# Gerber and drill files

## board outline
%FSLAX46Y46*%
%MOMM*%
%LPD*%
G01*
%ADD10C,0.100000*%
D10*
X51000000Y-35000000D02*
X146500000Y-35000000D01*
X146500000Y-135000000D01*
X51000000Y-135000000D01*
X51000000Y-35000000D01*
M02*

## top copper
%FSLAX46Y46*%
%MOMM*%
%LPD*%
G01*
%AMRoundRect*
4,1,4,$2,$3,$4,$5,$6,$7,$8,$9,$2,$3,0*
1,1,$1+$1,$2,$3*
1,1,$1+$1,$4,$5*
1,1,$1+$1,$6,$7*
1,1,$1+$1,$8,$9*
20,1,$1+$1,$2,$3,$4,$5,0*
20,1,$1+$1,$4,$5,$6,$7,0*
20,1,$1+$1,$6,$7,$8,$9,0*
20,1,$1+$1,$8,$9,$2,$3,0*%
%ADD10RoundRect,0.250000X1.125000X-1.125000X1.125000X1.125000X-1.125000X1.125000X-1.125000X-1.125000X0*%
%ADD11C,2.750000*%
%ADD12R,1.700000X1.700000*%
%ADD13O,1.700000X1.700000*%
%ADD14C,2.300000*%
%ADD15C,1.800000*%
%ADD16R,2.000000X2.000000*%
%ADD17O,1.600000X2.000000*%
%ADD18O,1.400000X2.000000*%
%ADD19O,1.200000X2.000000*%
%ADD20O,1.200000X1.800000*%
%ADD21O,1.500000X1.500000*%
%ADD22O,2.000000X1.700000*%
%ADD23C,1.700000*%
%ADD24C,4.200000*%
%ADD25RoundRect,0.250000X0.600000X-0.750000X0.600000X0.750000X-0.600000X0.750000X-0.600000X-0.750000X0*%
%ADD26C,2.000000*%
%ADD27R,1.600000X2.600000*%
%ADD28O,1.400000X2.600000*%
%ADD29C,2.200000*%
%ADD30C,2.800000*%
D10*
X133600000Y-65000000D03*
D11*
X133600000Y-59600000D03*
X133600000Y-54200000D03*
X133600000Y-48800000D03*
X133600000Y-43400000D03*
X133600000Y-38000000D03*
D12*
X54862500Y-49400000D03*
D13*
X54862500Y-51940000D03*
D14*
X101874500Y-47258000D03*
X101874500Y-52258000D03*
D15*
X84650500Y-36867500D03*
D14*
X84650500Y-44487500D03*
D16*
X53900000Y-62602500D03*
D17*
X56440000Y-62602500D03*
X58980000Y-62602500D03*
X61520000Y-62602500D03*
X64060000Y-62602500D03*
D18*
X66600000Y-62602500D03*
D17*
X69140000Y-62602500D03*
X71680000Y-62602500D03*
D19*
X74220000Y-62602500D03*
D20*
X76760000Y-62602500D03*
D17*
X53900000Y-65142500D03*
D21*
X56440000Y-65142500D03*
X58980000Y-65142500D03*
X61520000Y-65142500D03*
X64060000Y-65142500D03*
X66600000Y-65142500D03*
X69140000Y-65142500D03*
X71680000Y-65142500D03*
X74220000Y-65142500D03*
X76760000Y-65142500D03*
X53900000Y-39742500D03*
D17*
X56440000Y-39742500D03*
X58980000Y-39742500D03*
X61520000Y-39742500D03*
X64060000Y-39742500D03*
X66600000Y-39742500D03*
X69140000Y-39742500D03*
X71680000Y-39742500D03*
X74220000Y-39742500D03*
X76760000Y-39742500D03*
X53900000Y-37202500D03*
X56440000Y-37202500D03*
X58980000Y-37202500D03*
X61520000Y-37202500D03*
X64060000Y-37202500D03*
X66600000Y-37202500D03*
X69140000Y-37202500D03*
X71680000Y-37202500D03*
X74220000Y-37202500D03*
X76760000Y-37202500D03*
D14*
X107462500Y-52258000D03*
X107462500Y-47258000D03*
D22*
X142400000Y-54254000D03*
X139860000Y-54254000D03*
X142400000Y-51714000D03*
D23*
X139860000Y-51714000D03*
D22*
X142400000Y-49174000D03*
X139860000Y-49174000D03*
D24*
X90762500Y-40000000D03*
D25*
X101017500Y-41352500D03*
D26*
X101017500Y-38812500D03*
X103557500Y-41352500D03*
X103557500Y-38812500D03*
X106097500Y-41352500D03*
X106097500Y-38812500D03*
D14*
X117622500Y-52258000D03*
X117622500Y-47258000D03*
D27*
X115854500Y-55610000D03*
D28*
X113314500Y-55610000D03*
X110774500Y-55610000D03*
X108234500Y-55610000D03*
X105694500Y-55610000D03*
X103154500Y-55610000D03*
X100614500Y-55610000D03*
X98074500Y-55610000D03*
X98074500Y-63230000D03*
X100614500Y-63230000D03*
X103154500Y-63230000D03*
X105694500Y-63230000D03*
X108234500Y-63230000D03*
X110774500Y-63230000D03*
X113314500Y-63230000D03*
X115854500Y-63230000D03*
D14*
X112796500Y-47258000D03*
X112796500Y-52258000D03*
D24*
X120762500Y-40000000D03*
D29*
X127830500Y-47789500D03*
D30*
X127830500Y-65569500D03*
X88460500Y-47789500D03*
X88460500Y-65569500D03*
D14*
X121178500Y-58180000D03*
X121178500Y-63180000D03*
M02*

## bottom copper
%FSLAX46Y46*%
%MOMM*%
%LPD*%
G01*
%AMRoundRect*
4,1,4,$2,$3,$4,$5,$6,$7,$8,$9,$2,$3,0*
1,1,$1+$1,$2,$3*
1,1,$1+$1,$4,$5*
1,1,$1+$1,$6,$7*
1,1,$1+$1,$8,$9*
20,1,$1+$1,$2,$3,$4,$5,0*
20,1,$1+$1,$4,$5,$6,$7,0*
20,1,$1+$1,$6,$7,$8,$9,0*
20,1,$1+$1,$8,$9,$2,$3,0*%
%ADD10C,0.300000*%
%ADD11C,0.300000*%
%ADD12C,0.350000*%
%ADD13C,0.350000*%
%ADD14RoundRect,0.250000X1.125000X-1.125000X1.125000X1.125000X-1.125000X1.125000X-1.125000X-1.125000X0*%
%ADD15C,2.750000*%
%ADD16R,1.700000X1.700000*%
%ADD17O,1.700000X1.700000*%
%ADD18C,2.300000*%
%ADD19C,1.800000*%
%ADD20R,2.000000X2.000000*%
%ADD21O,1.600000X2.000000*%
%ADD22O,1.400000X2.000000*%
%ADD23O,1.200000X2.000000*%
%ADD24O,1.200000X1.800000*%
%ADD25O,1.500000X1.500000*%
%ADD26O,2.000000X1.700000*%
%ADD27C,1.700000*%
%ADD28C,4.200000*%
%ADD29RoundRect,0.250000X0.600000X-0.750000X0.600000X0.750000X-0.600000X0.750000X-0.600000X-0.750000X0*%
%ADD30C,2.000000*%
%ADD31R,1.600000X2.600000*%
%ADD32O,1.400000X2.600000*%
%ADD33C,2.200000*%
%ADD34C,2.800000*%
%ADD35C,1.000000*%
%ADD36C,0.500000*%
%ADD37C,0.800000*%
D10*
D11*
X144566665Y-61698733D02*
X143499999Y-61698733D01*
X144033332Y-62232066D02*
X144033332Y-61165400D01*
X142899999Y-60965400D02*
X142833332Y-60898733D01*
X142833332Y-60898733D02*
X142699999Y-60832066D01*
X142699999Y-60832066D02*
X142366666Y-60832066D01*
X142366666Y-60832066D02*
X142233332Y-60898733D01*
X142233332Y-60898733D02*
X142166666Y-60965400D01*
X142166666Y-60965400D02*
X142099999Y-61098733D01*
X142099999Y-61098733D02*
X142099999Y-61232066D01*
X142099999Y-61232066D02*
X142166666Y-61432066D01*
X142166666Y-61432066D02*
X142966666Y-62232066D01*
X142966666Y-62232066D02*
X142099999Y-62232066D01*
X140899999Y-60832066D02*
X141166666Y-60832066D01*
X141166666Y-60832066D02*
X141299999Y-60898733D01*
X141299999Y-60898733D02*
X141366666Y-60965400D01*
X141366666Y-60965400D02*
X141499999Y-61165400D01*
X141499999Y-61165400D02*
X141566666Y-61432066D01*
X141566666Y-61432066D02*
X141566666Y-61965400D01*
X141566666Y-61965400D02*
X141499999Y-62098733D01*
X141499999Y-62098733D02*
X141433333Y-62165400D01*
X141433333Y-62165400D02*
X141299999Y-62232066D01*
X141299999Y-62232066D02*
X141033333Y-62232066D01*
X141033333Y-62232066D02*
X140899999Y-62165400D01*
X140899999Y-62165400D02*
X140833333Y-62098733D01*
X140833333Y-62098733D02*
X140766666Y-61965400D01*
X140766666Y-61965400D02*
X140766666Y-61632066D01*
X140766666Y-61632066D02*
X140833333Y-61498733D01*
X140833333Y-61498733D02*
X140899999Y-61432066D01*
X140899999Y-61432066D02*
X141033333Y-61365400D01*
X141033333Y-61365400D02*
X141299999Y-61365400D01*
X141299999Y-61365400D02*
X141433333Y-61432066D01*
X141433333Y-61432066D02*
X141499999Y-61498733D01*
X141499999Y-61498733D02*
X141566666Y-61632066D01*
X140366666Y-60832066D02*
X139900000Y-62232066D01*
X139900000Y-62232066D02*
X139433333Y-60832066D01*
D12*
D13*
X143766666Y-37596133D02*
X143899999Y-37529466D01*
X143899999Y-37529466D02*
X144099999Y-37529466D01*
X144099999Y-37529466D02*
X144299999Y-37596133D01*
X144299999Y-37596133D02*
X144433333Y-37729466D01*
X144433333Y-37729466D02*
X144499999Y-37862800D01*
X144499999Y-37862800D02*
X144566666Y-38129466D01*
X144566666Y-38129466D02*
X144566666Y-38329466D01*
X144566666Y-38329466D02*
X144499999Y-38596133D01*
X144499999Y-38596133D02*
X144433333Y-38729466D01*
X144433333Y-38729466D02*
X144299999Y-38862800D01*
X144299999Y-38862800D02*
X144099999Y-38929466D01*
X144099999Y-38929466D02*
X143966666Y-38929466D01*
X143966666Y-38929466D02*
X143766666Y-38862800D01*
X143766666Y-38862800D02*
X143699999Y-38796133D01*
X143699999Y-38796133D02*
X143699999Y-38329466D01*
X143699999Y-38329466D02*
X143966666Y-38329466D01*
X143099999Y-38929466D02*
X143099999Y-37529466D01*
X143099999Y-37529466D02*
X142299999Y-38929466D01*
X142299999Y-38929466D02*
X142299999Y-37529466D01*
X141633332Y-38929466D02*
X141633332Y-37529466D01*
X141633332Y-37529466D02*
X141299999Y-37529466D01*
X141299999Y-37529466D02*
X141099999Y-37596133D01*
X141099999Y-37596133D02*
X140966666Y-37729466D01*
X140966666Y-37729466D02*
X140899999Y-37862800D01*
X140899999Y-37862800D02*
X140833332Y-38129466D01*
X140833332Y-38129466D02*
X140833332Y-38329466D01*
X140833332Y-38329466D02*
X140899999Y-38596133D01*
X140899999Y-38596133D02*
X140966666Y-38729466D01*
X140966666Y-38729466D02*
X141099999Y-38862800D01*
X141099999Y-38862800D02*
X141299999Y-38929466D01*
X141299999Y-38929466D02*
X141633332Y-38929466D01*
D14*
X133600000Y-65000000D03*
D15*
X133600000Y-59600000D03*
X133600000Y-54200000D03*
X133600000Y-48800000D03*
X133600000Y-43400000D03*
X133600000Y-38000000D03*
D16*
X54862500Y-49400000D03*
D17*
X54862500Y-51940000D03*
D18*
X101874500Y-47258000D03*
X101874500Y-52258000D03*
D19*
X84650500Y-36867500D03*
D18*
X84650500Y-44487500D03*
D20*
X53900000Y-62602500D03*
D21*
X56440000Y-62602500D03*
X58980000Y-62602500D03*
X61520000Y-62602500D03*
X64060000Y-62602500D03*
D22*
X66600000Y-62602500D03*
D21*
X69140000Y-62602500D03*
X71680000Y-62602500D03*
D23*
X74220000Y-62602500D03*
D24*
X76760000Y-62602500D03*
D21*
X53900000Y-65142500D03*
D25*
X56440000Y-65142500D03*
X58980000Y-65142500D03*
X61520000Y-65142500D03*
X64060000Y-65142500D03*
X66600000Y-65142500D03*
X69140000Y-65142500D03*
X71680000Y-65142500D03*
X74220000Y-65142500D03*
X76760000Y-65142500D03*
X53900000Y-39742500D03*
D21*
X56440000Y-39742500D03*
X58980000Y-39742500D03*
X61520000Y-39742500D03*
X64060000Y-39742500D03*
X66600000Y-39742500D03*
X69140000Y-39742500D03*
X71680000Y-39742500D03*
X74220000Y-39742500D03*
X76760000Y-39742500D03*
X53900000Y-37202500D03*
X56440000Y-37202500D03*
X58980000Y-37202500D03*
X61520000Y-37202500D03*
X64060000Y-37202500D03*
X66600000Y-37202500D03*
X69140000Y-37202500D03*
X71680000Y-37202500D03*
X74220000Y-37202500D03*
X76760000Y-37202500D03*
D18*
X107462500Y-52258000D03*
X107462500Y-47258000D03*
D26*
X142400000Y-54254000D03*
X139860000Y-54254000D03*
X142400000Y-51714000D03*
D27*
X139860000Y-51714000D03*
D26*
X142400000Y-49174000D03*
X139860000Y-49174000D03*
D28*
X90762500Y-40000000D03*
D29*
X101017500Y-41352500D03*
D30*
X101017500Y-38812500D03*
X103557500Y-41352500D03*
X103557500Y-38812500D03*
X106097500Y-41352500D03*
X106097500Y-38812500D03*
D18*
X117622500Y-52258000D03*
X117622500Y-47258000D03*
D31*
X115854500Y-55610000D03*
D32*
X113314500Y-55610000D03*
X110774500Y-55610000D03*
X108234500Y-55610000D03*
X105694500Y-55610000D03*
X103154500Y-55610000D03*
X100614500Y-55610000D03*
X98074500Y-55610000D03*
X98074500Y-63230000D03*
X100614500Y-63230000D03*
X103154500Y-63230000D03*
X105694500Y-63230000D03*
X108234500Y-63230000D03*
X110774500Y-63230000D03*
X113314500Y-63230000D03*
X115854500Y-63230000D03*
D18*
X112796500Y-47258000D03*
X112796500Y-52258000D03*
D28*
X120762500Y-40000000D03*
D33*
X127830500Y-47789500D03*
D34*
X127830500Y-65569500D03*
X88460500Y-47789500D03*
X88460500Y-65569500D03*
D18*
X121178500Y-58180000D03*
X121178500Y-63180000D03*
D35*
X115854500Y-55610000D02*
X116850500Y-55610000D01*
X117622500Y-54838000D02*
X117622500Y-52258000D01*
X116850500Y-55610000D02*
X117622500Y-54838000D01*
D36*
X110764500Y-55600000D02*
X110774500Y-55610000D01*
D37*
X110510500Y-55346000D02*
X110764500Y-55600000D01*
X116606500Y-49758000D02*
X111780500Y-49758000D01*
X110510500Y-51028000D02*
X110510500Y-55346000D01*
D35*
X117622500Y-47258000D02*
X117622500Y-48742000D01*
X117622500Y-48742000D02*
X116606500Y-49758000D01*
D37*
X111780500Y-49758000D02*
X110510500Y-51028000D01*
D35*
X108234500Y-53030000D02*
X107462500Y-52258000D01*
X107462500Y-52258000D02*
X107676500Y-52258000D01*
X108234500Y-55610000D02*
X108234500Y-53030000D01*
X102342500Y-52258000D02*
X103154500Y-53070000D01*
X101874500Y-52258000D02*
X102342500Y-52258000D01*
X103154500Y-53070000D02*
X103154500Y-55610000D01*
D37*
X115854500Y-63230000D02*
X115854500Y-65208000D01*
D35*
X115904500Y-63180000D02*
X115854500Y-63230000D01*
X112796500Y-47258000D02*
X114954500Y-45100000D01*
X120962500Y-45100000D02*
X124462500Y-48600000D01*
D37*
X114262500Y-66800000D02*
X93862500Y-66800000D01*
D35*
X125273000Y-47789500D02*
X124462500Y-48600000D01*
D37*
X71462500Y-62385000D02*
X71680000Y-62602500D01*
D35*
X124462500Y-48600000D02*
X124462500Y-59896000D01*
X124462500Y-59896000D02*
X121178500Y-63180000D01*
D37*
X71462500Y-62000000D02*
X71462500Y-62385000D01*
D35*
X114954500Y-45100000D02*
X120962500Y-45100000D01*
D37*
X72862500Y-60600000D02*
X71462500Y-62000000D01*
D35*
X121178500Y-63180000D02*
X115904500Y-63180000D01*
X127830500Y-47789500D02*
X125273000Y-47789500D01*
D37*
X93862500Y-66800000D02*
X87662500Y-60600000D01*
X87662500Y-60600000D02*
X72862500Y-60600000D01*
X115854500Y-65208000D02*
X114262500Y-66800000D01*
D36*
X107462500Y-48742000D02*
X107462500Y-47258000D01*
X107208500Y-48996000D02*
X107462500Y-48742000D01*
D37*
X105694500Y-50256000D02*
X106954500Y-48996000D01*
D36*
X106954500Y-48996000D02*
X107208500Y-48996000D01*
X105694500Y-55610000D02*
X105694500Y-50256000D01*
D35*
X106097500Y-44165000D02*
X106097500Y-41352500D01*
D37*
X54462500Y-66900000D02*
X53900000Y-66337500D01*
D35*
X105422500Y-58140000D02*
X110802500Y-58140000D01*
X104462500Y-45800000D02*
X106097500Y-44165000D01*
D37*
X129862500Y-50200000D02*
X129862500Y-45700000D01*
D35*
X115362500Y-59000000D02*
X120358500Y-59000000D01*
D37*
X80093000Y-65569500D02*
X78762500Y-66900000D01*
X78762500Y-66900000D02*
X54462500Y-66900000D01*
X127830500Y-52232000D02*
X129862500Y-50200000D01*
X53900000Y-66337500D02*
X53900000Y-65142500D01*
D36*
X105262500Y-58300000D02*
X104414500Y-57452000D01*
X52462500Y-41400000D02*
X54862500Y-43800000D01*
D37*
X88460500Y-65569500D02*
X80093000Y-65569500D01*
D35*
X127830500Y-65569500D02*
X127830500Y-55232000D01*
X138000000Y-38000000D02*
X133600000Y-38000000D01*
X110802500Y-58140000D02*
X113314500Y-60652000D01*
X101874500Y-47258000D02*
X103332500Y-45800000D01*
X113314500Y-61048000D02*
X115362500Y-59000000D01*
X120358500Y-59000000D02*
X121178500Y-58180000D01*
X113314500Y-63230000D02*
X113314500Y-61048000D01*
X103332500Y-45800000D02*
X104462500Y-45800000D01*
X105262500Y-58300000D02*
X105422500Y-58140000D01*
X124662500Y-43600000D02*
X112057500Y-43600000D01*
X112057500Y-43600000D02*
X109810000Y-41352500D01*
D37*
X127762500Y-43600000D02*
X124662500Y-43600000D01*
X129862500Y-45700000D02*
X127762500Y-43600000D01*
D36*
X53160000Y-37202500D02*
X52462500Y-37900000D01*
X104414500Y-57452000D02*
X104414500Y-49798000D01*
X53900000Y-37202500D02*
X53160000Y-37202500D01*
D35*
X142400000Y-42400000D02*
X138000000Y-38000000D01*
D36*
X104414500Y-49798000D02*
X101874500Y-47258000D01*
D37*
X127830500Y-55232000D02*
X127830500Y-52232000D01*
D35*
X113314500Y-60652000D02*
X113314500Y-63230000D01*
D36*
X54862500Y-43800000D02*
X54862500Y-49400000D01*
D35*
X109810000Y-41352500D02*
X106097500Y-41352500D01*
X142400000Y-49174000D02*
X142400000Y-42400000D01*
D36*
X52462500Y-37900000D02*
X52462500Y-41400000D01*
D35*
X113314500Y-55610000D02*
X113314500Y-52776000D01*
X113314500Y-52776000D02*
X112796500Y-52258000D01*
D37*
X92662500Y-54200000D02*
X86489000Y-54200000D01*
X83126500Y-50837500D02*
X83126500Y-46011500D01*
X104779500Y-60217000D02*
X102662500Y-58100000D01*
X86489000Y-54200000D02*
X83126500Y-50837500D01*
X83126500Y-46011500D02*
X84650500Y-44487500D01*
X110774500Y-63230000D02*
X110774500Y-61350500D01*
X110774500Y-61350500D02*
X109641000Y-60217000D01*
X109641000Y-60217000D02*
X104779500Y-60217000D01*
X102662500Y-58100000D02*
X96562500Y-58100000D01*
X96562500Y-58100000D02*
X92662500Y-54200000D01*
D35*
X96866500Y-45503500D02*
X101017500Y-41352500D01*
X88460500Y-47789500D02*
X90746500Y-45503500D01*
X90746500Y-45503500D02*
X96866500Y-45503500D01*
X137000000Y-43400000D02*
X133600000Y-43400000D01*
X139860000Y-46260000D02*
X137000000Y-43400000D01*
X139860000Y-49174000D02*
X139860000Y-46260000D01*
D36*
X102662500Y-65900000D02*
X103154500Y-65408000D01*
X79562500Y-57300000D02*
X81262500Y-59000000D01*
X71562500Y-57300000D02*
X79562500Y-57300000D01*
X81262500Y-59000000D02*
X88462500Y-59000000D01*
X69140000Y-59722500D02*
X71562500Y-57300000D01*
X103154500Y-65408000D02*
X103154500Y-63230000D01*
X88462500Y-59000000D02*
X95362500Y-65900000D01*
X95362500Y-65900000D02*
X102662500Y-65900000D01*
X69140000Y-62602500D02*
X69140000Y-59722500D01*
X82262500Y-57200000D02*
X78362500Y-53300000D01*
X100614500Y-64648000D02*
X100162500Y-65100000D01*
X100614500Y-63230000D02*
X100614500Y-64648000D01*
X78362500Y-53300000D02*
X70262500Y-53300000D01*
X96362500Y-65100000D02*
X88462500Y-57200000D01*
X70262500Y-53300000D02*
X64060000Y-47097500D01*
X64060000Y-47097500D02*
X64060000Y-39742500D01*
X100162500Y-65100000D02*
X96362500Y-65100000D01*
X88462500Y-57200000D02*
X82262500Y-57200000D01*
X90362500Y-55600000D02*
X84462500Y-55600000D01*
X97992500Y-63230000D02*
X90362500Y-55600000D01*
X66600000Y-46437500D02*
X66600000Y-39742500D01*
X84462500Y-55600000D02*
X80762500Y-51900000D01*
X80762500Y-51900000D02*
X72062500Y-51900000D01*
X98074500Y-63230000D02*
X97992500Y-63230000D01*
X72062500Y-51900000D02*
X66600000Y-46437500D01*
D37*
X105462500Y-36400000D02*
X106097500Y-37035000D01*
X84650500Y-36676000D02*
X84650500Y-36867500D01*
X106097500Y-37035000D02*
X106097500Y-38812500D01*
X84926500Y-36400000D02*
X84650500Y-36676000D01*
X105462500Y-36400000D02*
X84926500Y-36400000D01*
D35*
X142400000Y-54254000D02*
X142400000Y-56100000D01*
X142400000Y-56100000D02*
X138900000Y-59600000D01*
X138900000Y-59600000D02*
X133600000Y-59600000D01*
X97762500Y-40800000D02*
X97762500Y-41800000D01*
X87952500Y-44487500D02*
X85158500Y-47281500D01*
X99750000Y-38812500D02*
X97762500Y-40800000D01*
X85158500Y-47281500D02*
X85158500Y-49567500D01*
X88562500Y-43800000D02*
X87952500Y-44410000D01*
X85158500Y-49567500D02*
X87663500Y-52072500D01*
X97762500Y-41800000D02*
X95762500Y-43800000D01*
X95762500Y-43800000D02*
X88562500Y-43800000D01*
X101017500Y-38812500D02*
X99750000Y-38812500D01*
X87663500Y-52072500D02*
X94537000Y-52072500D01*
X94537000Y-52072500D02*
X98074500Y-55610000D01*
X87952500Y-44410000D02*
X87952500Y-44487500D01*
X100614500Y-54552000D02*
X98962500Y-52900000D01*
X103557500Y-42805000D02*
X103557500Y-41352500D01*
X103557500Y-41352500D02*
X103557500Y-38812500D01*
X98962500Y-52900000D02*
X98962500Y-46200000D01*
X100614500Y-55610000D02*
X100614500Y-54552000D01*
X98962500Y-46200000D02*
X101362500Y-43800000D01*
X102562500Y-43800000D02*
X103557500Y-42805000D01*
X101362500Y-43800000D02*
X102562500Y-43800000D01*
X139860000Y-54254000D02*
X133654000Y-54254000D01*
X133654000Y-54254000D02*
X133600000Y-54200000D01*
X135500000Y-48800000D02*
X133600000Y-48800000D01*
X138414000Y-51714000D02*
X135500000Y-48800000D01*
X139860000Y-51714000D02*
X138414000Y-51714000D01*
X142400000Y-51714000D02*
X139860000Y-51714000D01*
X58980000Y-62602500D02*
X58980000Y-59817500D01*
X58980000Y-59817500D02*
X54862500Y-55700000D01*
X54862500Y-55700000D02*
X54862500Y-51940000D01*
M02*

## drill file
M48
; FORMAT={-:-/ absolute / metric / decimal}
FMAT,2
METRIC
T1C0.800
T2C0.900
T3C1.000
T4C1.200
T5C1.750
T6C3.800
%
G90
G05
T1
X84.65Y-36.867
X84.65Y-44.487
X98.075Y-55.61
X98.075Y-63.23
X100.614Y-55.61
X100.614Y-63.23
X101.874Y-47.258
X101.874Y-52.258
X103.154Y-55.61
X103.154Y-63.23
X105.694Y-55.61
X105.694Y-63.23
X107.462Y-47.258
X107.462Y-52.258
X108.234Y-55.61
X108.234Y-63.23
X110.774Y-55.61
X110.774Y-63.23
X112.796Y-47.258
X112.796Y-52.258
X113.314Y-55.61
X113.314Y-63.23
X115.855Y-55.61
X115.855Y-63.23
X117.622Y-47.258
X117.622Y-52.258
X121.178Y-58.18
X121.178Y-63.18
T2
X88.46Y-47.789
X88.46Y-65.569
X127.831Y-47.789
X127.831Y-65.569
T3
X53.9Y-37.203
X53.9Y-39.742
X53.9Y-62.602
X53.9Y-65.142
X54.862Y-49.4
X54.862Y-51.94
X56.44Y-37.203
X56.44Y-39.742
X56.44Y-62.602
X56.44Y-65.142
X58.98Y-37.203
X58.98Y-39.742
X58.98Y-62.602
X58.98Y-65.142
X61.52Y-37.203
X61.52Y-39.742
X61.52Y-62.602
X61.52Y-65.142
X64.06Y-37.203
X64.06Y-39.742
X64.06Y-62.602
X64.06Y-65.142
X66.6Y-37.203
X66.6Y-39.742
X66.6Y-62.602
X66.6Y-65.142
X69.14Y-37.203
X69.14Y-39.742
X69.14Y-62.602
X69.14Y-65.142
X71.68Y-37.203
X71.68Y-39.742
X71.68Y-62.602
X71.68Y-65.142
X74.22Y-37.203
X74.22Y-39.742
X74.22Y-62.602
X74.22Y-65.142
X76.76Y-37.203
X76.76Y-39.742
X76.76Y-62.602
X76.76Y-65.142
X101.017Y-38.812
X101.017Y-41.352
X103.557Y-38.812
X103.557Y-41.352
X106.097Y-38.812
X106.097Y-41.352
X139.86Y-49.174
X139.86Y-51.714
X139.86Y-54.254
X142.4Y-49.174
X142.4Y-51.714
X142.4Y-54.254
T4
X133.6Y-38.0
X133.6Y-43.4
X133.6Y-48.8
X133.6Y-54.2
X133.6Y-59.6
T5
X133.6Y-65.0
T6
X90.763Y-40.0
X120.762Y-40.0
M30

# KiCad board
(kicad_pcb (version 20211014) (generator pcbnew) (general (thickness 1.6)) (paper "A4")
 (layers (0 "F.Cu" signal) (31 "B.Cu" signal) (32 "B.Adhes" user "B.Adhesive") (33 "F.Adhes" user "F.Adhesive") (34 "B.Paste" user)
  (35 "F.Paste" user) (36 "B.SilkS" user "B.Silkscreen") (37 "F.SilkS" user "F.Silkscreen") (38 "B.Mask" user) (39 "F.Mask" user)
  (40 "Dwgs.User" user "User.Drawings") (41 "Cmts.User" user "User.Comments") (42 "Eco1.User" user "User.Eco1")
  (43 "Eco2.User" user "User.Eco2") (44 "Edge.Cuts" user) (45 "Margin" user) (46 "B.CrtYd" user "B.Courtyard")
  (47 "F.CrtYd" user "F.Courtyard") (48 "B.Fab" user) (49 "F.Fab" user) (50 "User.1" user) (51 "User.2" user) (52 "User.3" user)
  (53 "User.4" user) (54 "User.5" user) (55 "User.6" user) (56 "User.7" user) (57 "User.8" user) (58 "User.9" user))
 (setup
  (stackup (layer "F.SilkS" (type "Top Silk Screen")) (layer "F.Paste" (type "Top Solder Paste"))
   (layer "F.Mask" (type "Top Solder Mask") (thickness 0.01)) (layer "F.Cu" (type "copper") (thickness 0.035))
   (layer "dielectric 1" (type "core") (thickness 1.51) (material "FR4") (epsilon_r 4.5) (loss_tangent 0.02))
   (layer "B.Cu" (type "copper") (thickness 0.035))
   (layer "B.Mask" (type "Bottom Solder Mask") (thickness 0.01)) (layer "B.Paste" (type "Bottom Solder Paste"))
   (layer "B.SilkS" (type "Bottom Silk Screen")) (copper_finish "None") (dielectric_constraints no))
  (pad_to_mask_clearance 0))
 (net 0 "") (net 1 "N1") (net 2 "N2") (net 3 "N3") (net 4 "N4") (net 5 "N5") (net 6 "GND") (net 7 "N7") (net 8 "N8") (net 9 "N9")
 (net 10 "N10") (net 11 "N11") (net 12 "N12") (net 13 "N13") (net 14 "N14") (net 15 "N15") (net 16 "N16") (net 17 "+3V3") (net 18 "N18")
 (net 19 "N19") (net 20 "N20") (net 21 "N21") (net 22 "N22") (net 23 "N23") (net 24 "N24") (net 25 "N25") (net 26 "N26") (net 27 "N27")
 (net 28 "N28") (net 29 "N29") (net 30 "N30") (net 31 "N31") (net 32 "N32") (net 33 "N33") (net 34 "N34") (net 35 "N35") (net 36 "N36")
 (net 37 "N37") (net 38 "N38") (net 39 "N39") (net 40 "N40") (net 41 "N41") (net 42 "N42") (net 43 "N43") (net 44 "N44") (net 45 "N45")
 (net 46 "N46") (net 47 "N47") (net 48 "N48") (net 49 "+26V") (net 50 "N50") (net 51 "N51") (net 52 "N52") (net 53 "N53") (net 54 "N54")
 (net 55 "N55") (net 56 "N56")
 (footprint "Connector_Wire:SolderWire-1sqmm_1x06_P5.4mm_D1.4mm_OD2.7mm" (layer "F.Cu") (at 133.6 65 90)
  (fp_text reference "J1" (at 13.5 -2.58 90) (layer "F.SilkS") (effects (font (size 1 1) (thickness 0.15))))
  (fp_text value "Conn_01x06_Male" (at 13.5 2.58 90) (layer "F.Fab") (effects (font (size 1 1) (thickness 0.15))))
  (pad "1" thru_hole roundrect (at 0 0 90) (size 2.75 2.75) (drill 1.75) (layers *.Cu *.Mask) (roundrect_rratio 0.090909) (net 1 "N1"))
  (pad "2" thru_hole circle (at 5.4 0 90) (size 2.75 2.75) (drill 1.2) (layers *.Cu *.Mask) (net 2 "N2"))
  (pad "3" thru_hole circle (at 10.8 0 90) (size 2.75 2.75) (drill 1.2) (layers *.Cu *.Mask) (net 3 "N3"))
  (pad "4" thru_hole circle (at 16.2 0 90) (size 2.75 2.75) (drill 1.2) (layers *.Cu *.Mask) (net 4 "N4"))
  (pad "5" thru_hole circle (at 21.6 0 90) (size 2.75 2.75) (drill 1.2) (layers *.Cu *.Mask) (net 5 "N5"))
  (pad "6" thru_hole circle (at 27 0 90) (size 2.75 2.75) (drill 1.2) (layers *.Cu *.Mask) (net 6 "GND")))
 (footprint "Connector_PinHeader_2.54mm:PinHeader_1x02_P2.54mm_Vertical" (layer "F.Cu") (at 54.8625 49.4)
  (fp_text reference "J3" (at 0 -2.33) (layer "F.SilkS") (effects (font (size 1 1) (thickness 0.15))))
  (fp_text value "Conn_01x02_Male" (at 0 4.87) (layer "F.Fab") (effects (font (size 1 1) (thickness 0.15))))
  (pad "1" thru_hole rect (at 0 0) (size 1.7 1.7) (drill 1) (layers *.Cu *.Mask) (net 6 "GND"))
  (pad "2" thru_hole oval (at 0 2.54) (size 1.7 1.7) (drill 1) (layers *.Cu *.Mask) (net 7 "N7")))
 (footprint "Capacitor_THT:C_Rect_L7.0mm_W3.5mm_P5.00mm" (layer "F.Cu") (at 101.8745 47.258 -90)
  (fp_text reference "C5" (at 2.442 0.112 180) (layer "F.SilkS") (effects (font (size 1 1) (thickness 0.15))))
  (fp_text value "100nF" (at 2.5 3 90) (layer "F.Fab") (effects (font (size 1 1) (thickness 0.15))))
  (pad "1" thru_hole circle (at 0 0 270) (size 2.3 2.3) (drill 0.8) (layers *.Cu *.Mask) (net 6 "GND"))
  (pad "2" thru_hole circle (at 5 0 270) (size 2.3 2.3) (drill 0.8) (layers *.Cu *.Mask) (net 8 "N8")))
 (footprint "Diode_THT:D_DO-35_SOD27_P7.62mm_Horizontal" (layer "F.Cu") (at 84.6505 36.8675 -90)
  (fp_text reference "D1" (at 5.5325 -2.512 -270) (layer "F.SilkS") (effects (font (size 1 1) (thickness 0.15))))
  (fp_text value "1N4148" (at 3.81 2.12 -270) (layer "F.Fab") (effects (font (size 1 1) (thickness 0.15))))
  (pad "1" thru_hole circle (at 0 0 270) (size 1.8 1.8) (drill 0.8) (layers *.Cu *.Mask) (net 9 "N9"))
  (pad "2" thru_hole circle (at 7.62 0 270) (size 2.3 2.3) (drill 0.8) (layers *.Cu *.Mask) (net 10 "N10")))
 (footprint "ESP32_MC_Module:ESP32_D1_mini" (layer "F.Cu") (at 53.9 65.1425 90)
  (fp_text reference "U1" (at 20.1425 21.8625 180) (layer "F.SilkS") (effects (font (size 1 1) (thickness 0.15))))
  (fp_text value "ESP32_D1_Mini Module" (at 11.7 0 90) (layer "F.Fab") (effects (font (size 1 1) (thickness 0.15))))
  (pad "1" thru_hole rect (at 2.54 0 90) (size 2 2) (drill 1) (layers *.Cu *.Mask) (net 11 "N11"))
  (pad "2" thru_hole oval (at 2.54 2.54 90) (size 2 1.6) (drill 1) (layers *.Cu *.Mask) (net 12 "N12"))
  (pad "3" thru_hole oval (at 2.54 5.08 90) (size 2 1.6) (drill 1) (layers *.Cu *.Mask) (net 7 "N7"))
  (pad "4" thru_hole oval (at 2.54 7.62 90) (size 2 1.6) (drill 1) (layers *.Cu *.Mask) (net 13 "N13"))
  (pad "5" thru_hole oval (at 2.54 10.16 90) (size 2 1.6) (drill 1) (layers *.Cu *.Mask) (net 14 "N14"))
  (pad "6" thru_hole oval (at 2.54 12.7 90) (size 2 1.4) (drill 1) (layers *.Cu *.Mask) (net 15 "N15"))
  (pad "7" thru_hole oval (at 2.54 15.24 90) (size 2 1.6) (drill 1) (layers *.Cu *.Mask) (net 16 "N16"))
  (pad "8" thru_hole oval (at 2.54 17.78 90) (size 2 1.6) (drill 1) (layers *.Cu *.Mask) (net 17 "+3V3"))
  (pad "9" thru_hole oval (at 2.54 20.32 90) (size 2 1.2) (drill 1) (layers *.Cu *.Mask) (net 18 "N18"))
  (pad "10" thru_hole oval (at 2.54 22.86 90) (size 1.8 1.2) (drill 1) (layers *.Cu *.Mask) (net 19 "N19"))
  (pad "11" thru_hole oval (at 0 0 90) (size 2 1.6) (drill 1) (layers *.Cu *.Mask) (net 6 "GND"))
  (pad "12" thru_hole oval (at 0 2.54 90) (size 1.5 1.5) (drill 1) (layers *.Cu *.Mask) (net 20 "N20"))
  (pad "13" thru_hole oval (at 0 5.08 90) (size 1.5 1.5) (drill 1) (layers *.Cu *.Mask) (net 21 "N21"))
  (pad "14" thru_hole oval (at 0 7.62 90) (size 1.5 1.5) (drill 1) (layers *.Cu *.Mask) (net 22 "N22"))
  (pad "15" thru_hole oval (at 0 10.16 90) (size 1.5 1.5) (drill 1) (layers *.Cu *.Mask) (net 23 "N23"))
  (pad "16" thru_hole oval (at 0 12.7 90) (size 1.5 1.5) (drill 1) (layers *.Cu *.Mask) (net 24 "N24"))
  (pad "17" thru_hole oval (at 0 15.24 90) (size 1.5 1.5) (drill 1) (layers *.Cu *.Mask) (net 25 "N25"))
  (pad "18" thru_hole oval (at 0 17.78 90) (size 1.5 1.5) (drill 1) (layers *.Cu *.Mask) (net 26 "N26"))
  (pad "19" thru_hole oval (at 0 20.32 90) (size 1.5 1.5) (drill 1) (layers *.Cu *.Mask) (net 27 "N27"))
  (pad "20" thru_hole oval (at 0 22.86 90) (size 1.5 1.5) (drill 1) (layers *.Cu *.Mask) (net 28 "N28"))
  (pad "21" thru_hole oval (at 25.4 0 90) (size 1.5 1.5) (drill 1) (layers *.Cu *.Mask) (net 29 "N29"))
  (pad "22" thru_hole oval (at 25.4 2.54 90) (size 2 1.6) (drill 1) (layers *.Cu *.Mask) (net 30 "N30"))
  (pad "23" thru_hole oval (at 25.4 5.08 90) (size 2 1.6) (drill 1) (layers *.Cu *.Mask) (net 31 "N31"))
  (pad "24" thru_hole oval (at 25.4 7.62 90) (size 2 1.6) (drill 1) (layers *.Cu *.Mask) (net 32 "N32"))
  (pad "25" thru_hole oval (at 25.4 10.16 90) (size 2 1.6) (drill 1) (layers *.Cu *.Mask) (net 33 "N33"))
  (pad "26" thru_hole oval (at 25.4 12.7 90) (size 2 1.6) (drill 1) (layers *.Cu *.Mask) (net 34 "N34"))
  (pad "27" thru_hole oval (at 25.4 15.24 90) (size 2 1.6) (drill 1) (layers *.Cu *.Mask) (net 6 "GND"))
  (pad "28" thru_hole oval (at 25.4 17.78 90) (size 2 1.6) (drill 1) (layers *.Cu *.Mask) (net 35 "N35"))
  (pad "29" thru_hole oval (at 25.4 20.32 90) (size 2 1.6) (drill 1) (layers *.Cu *.Mask) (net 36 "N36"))
  (pad "30" thru_hole oval (at 25.4 22.86 90) (size 2 1.6) (drill 1) (layers *.Cu *.Mask) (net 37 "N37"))
  (pad "31" thru_hole oval (at 27.94 0 90) (size 2 1.6) (drill 1) (layers *.Cu *.Mask) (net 6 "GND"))
  (pad "32" thru_hole oval (at 27.94 2.54 90) (size 2 1.6) (drill 1) (layers *.Cu *.Mask) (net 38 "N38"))
  (pad "33" thru_hole oval (at 27.94 5.08 90) (size 2 1.6) (drill 1) (layers *.Cu *.Mask) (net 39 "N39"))
  (pad "34" thru_hole oval (at 27.94 7.62 90) (size 2 1.6) (drill 1) (layers *.Cu *.Mask) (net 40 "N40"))
  (pad "35" thru_hole oval (at 27.94 10.16 90) (size 2 1.6) (drill 1) (layers *.Cu *.Mask) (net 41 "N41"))
  (pad "36" thru_hole oval (at 27.94 12.7 90) (size 2 1.6) (drill 1) (layers *.Cu *.Mask) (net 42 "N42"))
  (pad "37" thru_hole oval (at 27.94 15.24 90) (size 2 1.6) (drill 1) (layers *.Cu *.Mask) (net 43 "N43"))
  (pad "38" thru_hole oval (at 27.94 17.78 90) (size 2 1.6) (drill 1) (layers *.Cu *.Mask) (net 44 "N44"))
  (pad "39" thru_hole oval (at 27.94 20.32 90) (size 2 1.6) (drill 1) (layers *.Cu *.Mask) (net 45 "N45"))
  (pad "40" thru_hole oval (at 27.94 22.86 90) (size 2 1.6) (drill 1) (layers *.Cu *.Mask) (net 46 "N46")))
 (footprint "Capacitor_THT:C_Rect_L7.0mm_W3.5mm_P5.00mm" (layer "F.Cu") (at 107.4625 52.258 90)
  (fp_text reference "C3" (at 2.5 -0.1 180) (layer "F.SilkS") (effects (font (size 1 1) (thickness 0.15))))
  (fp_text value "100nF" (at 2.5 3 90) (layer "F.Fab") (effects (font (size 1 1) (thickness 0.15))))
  (pad "1" thru_hole circle (at 0 0 90) (size 2.3 2.3) (drill 0.8) (layers *.Cu *.Mask) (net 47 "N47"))
  (pad "2" thru_hole circle (at 5 0 90) (size 2.3 2.3) (drill 0.8) (layers *.Cu *.Mask) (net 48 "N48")))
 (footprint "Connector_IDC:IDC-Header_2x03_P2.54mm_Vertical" (layer "F.Cu") (at 142.4 54.254 180)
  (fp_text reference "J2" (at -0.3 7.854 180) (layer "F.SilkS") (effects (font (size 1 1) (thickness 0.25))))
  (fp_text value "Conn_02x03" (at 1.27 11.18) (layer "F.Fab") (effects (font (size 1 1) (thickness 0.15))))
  (pad "1" thru_hole oval (at 0 0 180) (size 2 1.7) (drill 1) (layers *.Cu *.Mask) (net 2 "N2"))
  (pad "2" thru_hole oval (at 2.54 0 180) (size 2 1.7) (drill 1) (layers *.Cu *.Mask) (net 3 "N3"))
  (pad "3" thru_hole oval (at 0 2.54 180) (size 2 1.7) (drill 1) (layers *.Cu *.Mask) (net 4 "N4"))
  (pad "4" thru_hole circle (at 2.54 2.54 180) (size 1.7 1.7) (drill 1) (layers *.Cu *.Mask) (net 4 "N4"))
  (pad "5" thru_hole oval (at 0 5.08 180) (size 2 1.7) (drill 1) (layers *.Cu *.Mask) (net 6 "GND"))
  (pad "6" thru_hole oval (at 2.54 5.08 180) (size 2 1.7) (drill 1) (layers *.Cu *.Mask) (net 5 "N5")))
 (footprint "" (layer "F.Cu") (at 90.7625 40)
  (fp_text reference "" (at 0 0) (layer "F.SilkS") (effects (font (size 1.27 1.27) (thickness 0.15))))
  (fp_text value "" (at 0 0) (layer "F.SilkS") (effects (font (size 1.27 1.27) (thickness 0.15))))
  (pad "1" thru_hole circle (at 0 0 270) (size 4.2 4.2) (drill 3.8) (layers *.Cu *.Mask) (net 17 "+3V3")))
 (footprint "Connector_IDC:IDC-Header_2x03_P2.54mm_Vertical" (layer "F.Cu") (at 101.0175 41.3525 90)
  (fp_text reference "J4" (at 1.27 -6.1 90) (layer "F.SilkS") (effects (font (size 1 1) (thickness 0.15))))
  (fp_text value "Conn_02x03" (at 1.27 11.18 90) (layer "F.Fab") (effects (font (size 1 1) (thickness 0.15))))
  (pad "1" thru_hole roundrect (at 0 0 90) (size 2 1.7) (drill 1) (layers *.Cu *.Mask) (roundrect_rratio 0.147059) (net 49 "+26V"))
  (pad "2" thru_hole circle (at 2.54 0 90) (size 2 2) (drill 1) (layers *.Cu *.Mask) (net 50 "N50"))
  (pad "3" thru_hole circle (at 0 2.54 90) (size 2 2) (drill 1) (layers *.Cu *.Mask) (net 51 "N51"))
  (pad "4" thru_hole circle (at 2.54 2.54 90) (size 2 2) (drill 1) (layers *.Cu *.Mask) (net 51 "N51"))
  (pad "5" thru_hole circle (at 0 5.08 90) (size 2 2) (drill 1) (layers *.Cu *.Mask) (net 6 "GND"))
  (pad "6" thru_hole circle (at 2.54 5.08 90) (size 2 2) (drill 1) (layers *.Cu *.Mask) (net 9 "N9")))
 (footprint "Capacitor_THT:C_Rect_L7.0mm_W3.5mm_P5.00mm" (layer "F.Cu") (at 117.6225 52.258 90)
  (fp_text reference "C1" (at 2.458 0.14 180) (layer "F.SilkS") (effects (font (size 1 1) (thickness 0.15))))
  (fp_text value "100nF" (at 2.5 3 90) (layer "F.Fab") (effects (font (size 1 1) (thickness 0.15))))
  (pad "1" thru_hole circle (at 0 0 90) (size 2.3 2.3) (drill 0.8) (layers *.Cu *.Mask) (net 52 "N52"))
  (pad "2" thru_hole circle (at 5 0 90) (size 2.3 2.3) (drill 0.8) (layers *.Cu *.Mask) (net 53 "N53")))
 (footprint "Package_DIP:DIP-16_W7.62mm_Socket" (layer "F.Cu") (at 115.8545 55.61 -90)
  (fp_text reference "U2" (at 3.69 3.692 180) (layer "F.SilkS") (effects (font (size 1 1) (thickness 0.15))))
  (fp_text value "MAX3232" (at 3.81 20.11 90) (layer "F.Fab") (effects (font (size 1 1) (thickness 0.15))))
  (pad "1" thru_hole rect (at 0 0 270) (size 2.6 1.6) (drill 0.8) (layers *.Cu *.Mask) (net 52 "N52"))
  (pad "2" thru_hole oval (at 0 2.54 270) (size 2.6 1.4) (drill 0.8) (layers *.Cu *.Mask) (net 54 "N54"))
  (pad "3" thru_hole oval (at 0 5.08 270) (size 2.6 1.4) (drill 0.8) (layers *.Cu *.Mask) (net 53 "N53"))
  (pad "4" thru_hole oval (at 0 7.62 270) (size 2.6 1.4) (drill 0.8) (layers *.Cu *.Mask) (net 47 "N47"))
  (pad "5" thru_hole oval (at 0 10.16 270) (size 2.6 1.4) (drill 0.8) (layers *.Cu *.Mask) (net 48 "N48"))
  (pad "6" thru_hole oval (at 0 12.7 270) (size 2.6 1.4) (drill 0.8) (layers *.Cu *.Mask) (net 8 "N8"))
  (pad "7" thru_hole oval (at 0 15.24 270) (size 2.6 1.4) (drill 0.8) (layers *.Cu *.Mask) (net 51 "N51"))
  (pad "8" thru_hole oval (at 0 17.78 270) (size 2.6 1.4) (drill 0.8) (layers *.Cu *.Mask) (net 50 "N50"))
  (pad "9" thru_hole oval (at 7.62 17.78 270) (size 2.6 1.4) (drill 0.8) (layers *.Cu *.Mask) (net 34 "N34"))
  (pad "10" thru_hole oval (at 7.62 15.24 270) (size 2.6 1.4) (drill 0.8) (layers *.Cu *.Mask) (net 33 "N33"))
  (pad "11" thru_hole oval (at 7.62 12.7 270) (size 2.6 1.4) (drill 0.8) (layers *.Cu *.Mask) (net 16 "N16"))
  (pad "12" thru_hole oval (at 7.62 10.16 270) (size 2.6 1.4) (drill 0.8) (layers *.Cu *.Mask) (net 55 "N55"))
  (pad "13" thru_hole oval (at 7.62 7.62 270) (size 2.6 1.4) (drill 0.8) (layers *.Cu *.Mask) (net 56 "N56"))
  (pad "14" thru_hole oval (at 7.62 5.08 270) (size 2.6 1.4) (drill 0.8) (layers *.Cu *.Mask) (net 10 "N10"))
  (pad "15" thru_hole oval (at 7.62 2.54 270) (size 2.6 1.4) (drill 0.8) (layers *.Cu *.Mask) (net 6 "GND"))
  (pad "16" thru_hole oval (at 7.62 0 270) (size 2.6 1.4) (drill 0.8) (layers *.Cu *.Mask) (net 17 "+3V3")))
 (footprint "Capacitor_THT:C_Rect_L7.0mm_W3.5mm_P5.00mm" (layer "F.Cu") (at 112.7965 47.258 -90)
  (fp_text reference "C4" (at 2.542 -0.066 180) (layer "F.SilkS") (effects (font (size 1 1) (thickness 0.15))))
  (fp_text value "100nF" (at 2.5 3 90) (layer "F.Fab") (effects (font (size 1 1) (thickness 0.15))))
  (pad "1" thru_hole circle (at 0 0 270) (size 2.3 2.3) (drill 0.8) (layers *.Cu *.Mask) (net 17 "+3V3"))
  (pad "2" thru_hole circle (at 5 0 270) (size 2.3 2.3) (drill 0.8) (layers *.Cu *.Mask) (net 54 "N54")))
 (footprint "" (layer "F.Cu") (at 120.7625 40)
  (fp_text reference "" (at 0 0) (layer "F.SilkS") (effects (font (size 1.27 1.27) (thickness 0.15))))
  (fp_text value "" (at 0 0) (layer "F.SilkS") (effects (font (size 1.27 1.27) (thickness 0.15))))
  (pad "1" thru_hole circle (at 0 0 270) (size 4.2 4.2) (drill 3.8) (layers *.Cu *.Mask) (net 17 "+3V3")))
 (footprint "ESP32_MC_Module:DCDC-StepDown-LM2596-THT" (layer "F.Cu") (at 127.8305 47.7895 -90)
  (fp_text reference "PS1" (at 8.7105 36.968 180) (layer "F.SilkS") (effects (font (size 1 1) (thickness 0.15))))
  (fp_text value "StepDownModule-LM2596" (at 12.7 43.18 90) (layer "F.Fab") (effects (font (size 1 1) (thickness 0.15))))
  (pad "1" thru_hole circle (at 0 0 270) (size 2.2 2.2) (drill 0.9) (layers *.Cu *.Mask) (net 17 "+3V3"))
  (pad "2" thru_hole circle (at 17.78 0 270) (size 2.8 2.8) (drill 0.9) (layers *.Cu *.Mask) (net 6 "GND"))
  (pad "3" thru_hole circle (at 0 39.37 270) (size 2.8 2.8) (drill 0.9) (layers *.Cu *.Mask) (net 49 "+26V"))
  (pad "4" thru_hole circle (at 17.78 39.37 270) (size 2.8 2.8) (drill 0.9) (layers *.Cu *.Mask) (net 6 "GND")))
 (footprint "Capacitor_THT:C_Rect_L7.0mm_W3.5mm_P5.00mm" (layer "F.Cu") (at 121.1785 58.18 -90)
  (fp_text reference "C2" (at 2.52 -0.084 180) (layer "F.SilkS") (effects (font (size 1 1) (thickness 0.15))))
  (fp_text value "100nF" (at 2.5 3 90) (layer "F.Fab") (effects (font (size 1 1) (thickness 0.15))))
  (pad "1" thru_hole circle (at 0 0 270) (size 2.3 2.3) (drill 0.8) (layers *.Cu *.Mask) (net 6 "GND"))
  (pad "2" thru_hole circle (at 5 0 270) (size 2.3 2.3) (drill 0.8) (layers *.Cu *.Mask) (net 17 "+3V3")))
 (gr_rect (start 51 35) (end 146.5 135) (layer "Edge.Cuts") (width 0.1) (fill none))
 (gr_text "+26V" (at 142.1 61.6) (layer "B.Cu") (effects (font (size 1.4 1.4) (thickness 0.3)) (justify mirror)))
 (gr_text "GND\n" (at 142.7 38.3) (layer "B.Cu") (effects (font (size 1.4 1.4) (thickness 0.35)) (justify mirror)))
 (segment (start 115.8545 55.61) (end 116.8505 55.61) (width 1) (layer "B.Cu") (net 52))
 (segment (start 117.6225 54.838) (end 117.6225 52.258) (width 1) (layer "B.Cu") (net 52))
 (segment (start 116.8505 55.61) (end 117.6225 54.838) (width 1) (layer "B.Cu") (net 52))
 (segment (start 110.7645 55.6) (end 110.7745 55.61) (width 0.5) (layer "B.Cu") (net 53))
 (segment (start 110.5105 55.346) (end 110.7645 55.6) (width 0.8) (layer "B.Cu") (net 53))
 (segment (start 116.6065 49.758) (end 111.7805 49.758) (width 0.8) (layer "B.Cu") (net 53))
 (segment (start 110.5105 51.028) (end 110.5105 55.346) (width 0.8) (layer "B.Cu") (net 53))
 (segment (start 117.6225 47.258) (end 117.6225 48.742) (width 1) (layer "B.Cu") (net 53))
 (segment (start 117.6225 48.742) (end 116.6065 49.758) (width 1) (layer "B.Cu") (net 53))
 (segment (start 111.7805 49.758) (end 110.5105 51.028) (width 0.8) (layer "B.Cu") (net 53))
 (segment (start 108.2345 53.03) (end 107.4625 52.258) (width 1) (layer "B.Cu") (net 47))
 (segment (start 107.4625 52.258) (end 107.6765 52.258) (width 1) (layer "B.Cu") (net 47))
 (segment (start 108.2345 55.61) (end 108.2345 53.03) (width 1) (layer "B.Cu") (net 47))
 (segment (start 102.3425 52.258) (end 103.1545 53.07) (width 1) (layer "B.Cu") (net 8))
 (segment (start 101.8745 52.258) (end 102.3425 52.258) (width 1) (layer "B.Cu") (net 8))
 (segment (start 103.1545 53.07) (end 103.1545 55.61) (width 1) (layer "B.Cu") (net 8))
 (segment (start 115.8545 63.23) (end 115.8545 65.208) (width 0.8) (layer "B.Cu") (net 17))
 (segment (start 115.9045 63.18) (end 115.8545 63.23) (width 1) (layer "B.Cu") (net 17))
 (segment (start 112.7965 47.258) (end 114.9545 45.1) (width 1) (layer "B.Cu") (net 17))
 (segment (start 120.9625 45.1) (end 124.4625 48.6) (width 1) (layer "B.Cu") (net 17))
 (segment (start 114.2625 66.8) (end 93.8625 66.8) (width 0.8) (layer "B.Cu") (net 17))
 (segment (start 125.273 47.7895) (end 124.4625 48.6) (width 1) (layer "B.Cu") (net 17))
 (segment (start 71.4625 62.385) (end 71.68 62.6025) (width 0.8) (layer "B.Cu") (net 17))
 (segment (start 124.4625 48.6) (end 124.4625 59.896) (width 1) (layer "B.Cu") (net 17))
 (segment (start 124.4625 59.896) (end 121.1785 63.18) (width 1) (layer "B.Cu") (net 17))
 (segment (start 71.4625 62) (end 71.4625 62.385) (width 0.8) (layer "B.Cu") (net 17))
 (segment (start 114.9545 45.1) (end 120.9625 45.1) (width 1) (layer "B.Cu") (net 17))
 (segment (start 72.8625 60.6) (end 71.4625 62) (width 0.8) (layer "B.Cu") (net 17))
 (segment (start 121.1785 63.18) (end 115.9045 63.18) (width 1) (layer "B.Cu") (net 17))
 (segment (start 127.8305 47.7895) (end 125.273 47.7895) (width 1) (layer "B.Cu") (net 17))
 (segment (start 93.8625 66.8) (end 87.6625 60.6) (width 0.8) (layer "B.Cu") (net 17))
 (segment (start 87.6625 60.6) (end 72.8625 60.6) (width 0.8) (layer "B.Cu") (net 17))
 (segment (start 115.8545 65.208) (end 114.2625 66.8) (width 0.8) (layer "B.Cu") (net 17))
 (segment (start 107.4625 48.742) (end 107.4625 47.258) (width 0.5) (layer "B.Cu") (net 48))
 (segment (start 107.2085 48.996) (end 107.4625 48.742) (width 0.5) (layer "B.Cu") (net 48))
 (segment (start 105.6945 50.256) (end 106.9545 48.996) (width 0.8) (layer "B.Cu") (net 48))
 (segment (start 106.9545 48.996) (end 107.2085 48.996) (width 0.5) (layer "B.Cu") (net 48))
 (segment (start 105.6945 55.61) (end 105.6945 50.256) (width 0.5) (layer "B.Cu") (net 48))
 (segment (start 106.0975 44.165) (end 106.0975 41.3525) (width 1) (layer "B.Cu") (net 6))
 (segment (start 54.4625 66.9) (end 53.9 66.3375) (width 0.8) (layer "B.Cu") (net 6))
 (segment (start 105.4225 58.14) (end 110.8025 58.14) (width 1) (layer "B.Cu") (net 6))
 (segment (start 104.4625 45.8) (end 106.0975 44.165) (width 1) (layer "B.Cu") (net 6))
 (segment (start 129.8625 50.2) (end 129.8625 45.7) (width 0.8) (layer "B.Cu") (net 6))
 (segment (start 115.3625 59) (end 120.3585 59) (width 1) (layer "B.Cu") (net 6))
 (segment (start 80.093 65.5695) (end 78.7625 66.9) (width 0.8) (layer "B.Cu") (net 6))
 (segment (start 78.7625 66.9) (end 54.4625 66.9) (width 0.8) (layer "B.Cu") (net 6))
 (segment (start 127.8305 52.232) (end 129.8625 50.2) (width 0.8) (layer "B.Cu") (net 6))
 (segment (start 53.9 66.3375) (end 53.9 65.1425) (width 0.8) (layer "B.Cu") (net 6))
 (segment (start 105.2625 58.3) (end 104.4145 57.452) (width 0.5) (layer "B.Cu") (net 6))
 (segment (start 52.4625 41.4) (end 54.8625 43.8) (width 0.5) (layer "B.Cu") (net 6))
 (segment (start 88.4605 65.5695) (end 80.093 65.5695) (width 0.8) (layer "B.Cu") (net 6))
 (segment (start 127.8305 65.5695) (end 127.8305 55.232) (width 1) (layer "B.Cu") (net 6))
 (segment (start 138 38) (end 133.6 38) (width 1) (layer "B.Cu") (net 6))
 (segment (start 110.8025 58.14) (end 113.3145 60.652) (width 1) (layer "B.Cu") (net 6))
 (segment (start 101.8745 47.258) (end 103.3325 45.8) (width 1) (layer "B.Cu") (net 6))
 (segment (start 113.3145 61.048) (end 115.3625 59) (width 1) (layer "B.Cu") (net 6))
 (segment (start 120.3585 59) (end 121.1785 58.18) (width 1) (layer "B.Cu") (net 6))
 (segment (start 113.3145 63.23) (end 113.3145 61.048) (width 1) (layer "B.Cu") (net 6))
 (segment (start 103.3325 45.8) (end 104.4625 45.8) (width 1) (layer "B.Cu") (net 6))
 (segment (start 105.2625 58.3) (end 105.4225 58.14) (width 1) (layer "B.Cu") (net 6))
 (segment (start 124.6625 43.6) (end 112.0575 43.6) (width 1) (layer "B.Cu") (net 6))
 (segment (start 112.0575 43.6) (end 109.81 41.3525) (width 1) (layer "B.Cu") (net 6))
 (segment (start 127.7625 43.6) (end 124.6625 43.6) (width 0.8) (layer "B.Cu") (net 6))
 (segment (start 129.8625 45.7) (end 127.7625 43.6) (width 0.8) (layer "B.Cu") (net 6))
 (segment (start 53.16 37.2025) (end 52.4625 37.9) (width 0.5) (layer "B.Cu") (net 6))
 (segment (start 104.4145 57.452) (end 104.4145 49.798) (width 0.5) (layer "B.Cu") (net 6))
 (segment (start 53.9 37.2025) (end 53.16 37.2025) (width 0.5) (layer "B.Cu") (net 6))
 (segment (start 142.4 42.4) (end 138 38) (width 1) (layer "B.Cu") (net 6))
 (segment (start 104.4145 49.798) (end 101.8745 47.258) (width 0.5) (layer "B.Cu") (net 6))
 (segment (start 127.8305 55.232) (end 127.8305 52.232) (width 0.8) (layer "B.Cu") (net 6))
 (segment (start 113.3145 60.652) (end 113.3145 63.23) (width 1) (layer "B.Cu") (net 6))
 (segment (start 54.8625 43.8) (end 54.8625 49.4) (width 0.5) (layer "B.Cu") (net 6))
 (segment (start 109.81 41.3525) (end 106.0975 41.3525) (width 1) (layer "B.Cu") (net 6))
 (segment (start 142.4 49.174) (end 142.4 42.4) (width 1) (layer "B.Cu") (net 6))
 (segment (start 52.4625 37.9) (end 52.4625 41.4) (width 0.5) (layer "B.Cu") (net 6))
 (segment (start 113.3145 55.61) (end 113.3145 52.776) (width 1) (layer "B.Cu") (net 54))
 (segment (start 113.3145 52.776) (end 112.7965 52.258) (width 1) (layer "B.Cu") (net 54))
 (segment (start 92.6625 54.2) (end 86.489 54.2) (width 0.8) (layer "B.Cu") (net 10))
 (segment (start 83.1265 50.8375) (end 83.1265 46.0115) (width 0.8) (layer "B.Cu") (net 10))
 (segment (start 104.7795 60.217) (end 102.6625 58.1) (width 0.8) (layer "B.Cu") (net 10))
 (segment (start 86.489 54.2) (end 83.1265 50.8375) (width 0.8) (layer "B.Cu") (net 10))
 (segment (start 83.1265 46.0115) (end 84.6505 44.4875) (width 0.8) (layer "B.Cu") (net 10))
 (segment (start 110.7745 63.23) (end 110.7745 61.3505) (width 0.8) (layer "B.Cu") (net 10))
 (segment (start 110.7745 61.3505) (end 109.641 60.217) (width 0.8) (layer "B.Cu") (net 10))
 (segment (start 109.641 60.217) (end 104.7795 60.217) (width 0.8) (layer "B.Cu") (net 10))
 (segment (start 102.6625 58.1) (end 96.5625 58.1) (width 0.8) (layer "B.Cu") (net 10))
 (segment (start 96.5625 58.1) (end 92.6625 54.2) (width 0.8) (layer "B.Cu") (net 10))
 (segment (start 96.8665 45.5035) (end 101.0175 41.3525) (width 1) (layer "B.Cu") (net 49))
 (segment (start 88.4605 47.7895) (end 90.7465 45.5035) (width 1) (layer "B.Cu") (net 49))
 (segment (start 90.7465 45.5035) (end 96.8665 45.5035) (width 1) (layer "B.Cu") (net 49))
 (segment (start 137 43.4) (end 133.6 43.4) (width 1) (layer "B.Cu") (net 5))
 (segment (start 139.86 46.26) (end 137 43.4) (width 1) (layer "B.Cu") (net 5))
 (segment (start 139.86 49.174) (end 139.86 46.26) (width 1) (layer "B.Cu") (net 5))
 (segment (start 102.6625 65.9) (end 103.1545 65.408) (width 0.5) (layer "B.Cu") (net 16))
 (segment (start 79.5625 57.3) (end 81.2625 59) (width 0.5) (layer "B.Cu") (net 16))
 (segment (start 71.5625 57.3) (end 79.5625 57.3) (width 0.5) (layer "B.Cu") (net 16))
 (segment (start 81.2625 59) (end 88.4625 59) (width 0.5) (layer "B.Cu") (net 16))
 (segment (start 69.14 59.7225) (end 71.5625 57.3) (width 0.5) (layer "B.Cu") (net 16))
 (segment (start 103.1545 65.408) (end 103.1545 63.23) (width 0.5) (layer "B.Cu") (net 16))
 (segment (start 88.4625 59) (end 95.3625 65.9) (width 0.5) (layer "B.Cu") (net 16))
 (segment (start 95.3625 65.9) (end 102.6625 65.9) (width 0.5) (layer "B.Cu") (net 16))
 (segment (start 69.14 62.6025) (end 69.14 59.7225) (width 0.5) (layer "B.Cu") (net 16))
 (segment (start 82.2625 57.2) (end 78.3625 53.3) (width 0.5) (layer "B.Cu") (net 33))
 (segment (start 100.6145 64.648) (end 100.1625 65.1) (width 0.5) (layer "B.Cu") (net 33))
 (segment (start 100.6145 63.23) (end 100.6145 64.648) (width 0.5) (layer "B.Cu") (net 33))
 (segment (start 78.3625 53.3) (end 70.2625 53.3) (width 0.5) (layer "B.Cu") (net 33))
 (segment (start 96.3625 65.1) (end 88.4625 57.2) (width 0.5) (layer "B.Cu") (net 33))
 (segment (start 70.2625 53.3) (end 64.06 47.0975) (width 0.5) (layer "B.Cu") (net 33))
 (segment (start 64.06 47.0975) (end 64.06 39.7425) (width 0.5) (layer "B.Cu") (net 33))
 (segment (start 100.1625 65.1) (end 96.3625 65.1) (width 0.5) (layer "B.Cu") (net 33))
 (segment (start 88.4625 57.2) (end 82.2625 57.2) (width 0.5) (layer "B.Cu") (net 33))
 (segment (start 90.3625 55.6) (end 84.4625 55.6) (width 0.5) (layer "B.Cu") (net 34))
 (segment (start 97.9925 63.23) (end 90.3625 55.6) (width 0.5) (layer "B.Cu") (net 34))
 (segment (start 66.6 46.4375) (end 66.6 39.7425) (width 0.5) (layer "B.Cu") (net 34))
 (segment (start 84.4625 55.6) (end 80.7625 51.9) (width 0.5) (layer "B.Cu") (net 34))
 (segment (start 80.7625 51.9) (end 72.0625 51.9) (width 0.5) (layer "B.Cu") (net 34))
 (segment (start 98.0745 63.23) (end 97.9925 63.23) (width 0.5) (layer "B.Cu") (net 34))
 (segment (start 72.0625 51.9) (end 66.6 46.4375) (width 0.5) (layer "B.Cu") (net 34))
 (segment (start 105.4625 36.4) (end 106.0975 37.035) (width 0.8) (layer "B.Cu") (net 9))
 (segment (start 84.6505 36.676) (end 84.6505 36.8675) (width 0.8) (layer "B.Cu") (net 9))
 (segment (start 106.0975 37.035) (end 106.0975 38.8125) (width 0.8) (layer "B.Cu") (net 9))
 (segment (start 84.9265 36.4) (end 84.6505 36.676) (width 0.8) (layer "B.Cu") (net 9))
 (segment (start 105.4625 36.4) (end 84.9265 36.4) (width 0.8) (layer "B.Cu") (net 9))
 (segment (start 142.4 54.254) (end 142.4 56.1) (width 1) (layer "B.Cu") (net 2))
 (segment (start 142.4 56.1) (end 138.9 59.6) (width 1) (layer "B.Cu") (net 2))
 (segment (start 138.9 59.6) (end 133.6 59.6) (width 1) (layer "B.Cu") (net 2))
 (segment (start 97.7625 40.8) (end 97.7625 41.8) (width 1) (layer "B.Cu") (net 50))
 (segment (start 87.9525 44.4875) (end 85.1585 47.2815) (width 1) (layer "B.Cu") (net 50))
 (segment (start 99.75 38.8125) (end 97.7625 40.8) (width 1) (layer "B.Cu") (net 50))
 (segment (start 85.1585 47.2815) (end 85.1585 49.5675) (width 1) (layer "B.Cu") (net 50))
 (segment (start 88.5625 43.8) (end 87.9525 44.41) (width 1) (layer "B.Cu") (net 50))
 (segment (start 85.1585 49.5675) (end 87.6635 52.0725) (width 1) (layer "B.Cu") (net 50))
 (segment (start 97.7625 41.8) (end 95.7625 43.8) (width 1) (layer "B.Cu") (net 50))
 (segment (start 95.7625 43.8) (end 88.5625 43.8) (width 1) (layer "B.Cu") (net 50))
 (segment (start 101.0175 38.8125) (end 99.75 38.8125) (width 1) (layer "B.Cu") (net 50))
 (segment (start 87.6635 52.0725) (end 94.537 52.0725) (width 1) (layer "B.Cu") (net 50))
 (segment (start 94.537 52.0725) (end 98.0745 55.61) (width 1) (layer "B.Cu") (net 50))
 (segment (start 87.9525 44.41) (end 87.9525 44.4875) (width 1) (layer "B.Cu") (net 50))
 (segment (start 100.6145 54.552) (end 98.9625 52.9) (width 1) (layer "B.Cu") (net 51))
 (segment (start 103.5575 42.805) (end 103.5575 41.3525) (width 1) (layer "B.Cu") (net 51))
 (segment (start 103.5575 41.3525) (end 103.5575 38.8125) (width 1) (layer "B.Cu") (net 51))
 (segment (start 98.9625 52.9) (end 98.9625 46.2) (width 1) (layer "B.Cu") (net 51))
 (segment (start 100.6145 55.61) (end 100.6145 54.552) (width 1) (layer "B.Cu") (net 51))
 (segment (start 98.9625 46.2) (end 101.3625 43.8) (width 1) (layer "B.Cu") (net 51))
 (segment (start 102.5625 43.8) (end 103.5575 42.805) (width 1) (layer "B.Cu") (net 51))
 (segment (start 101.3625 43.8) (end 102.5625 43.8) (width 1) (layer "B.Cu") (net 51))
 (segment (start 139.86 54.254) (end 133.654 54.254) (width 1) (layer "B.Cu") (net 3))
 (segment (start 133.654 54.254) (end 133.6 54.2) (width 1) (layer "B.Cu") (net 3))
 (segment (start 135.5 48.8) (end 133.6 48.8) (width 1) (layer "B.Cu") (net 4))
 (segment (start 138.414 51.714) (end 135.5 48.8) (width 1) (layer "B.Cu") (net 4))
 (segment (start 139.86 51.714) (end 138.414 51.714) (width 1) (layer "B.Cu") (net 4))
 (segment (start 142.4 51.714) (end 139.86 51.714) (width 1) (layer "B.Cu") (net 4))
 (segment (start 58.98 62.6025) (end 58.98 59.8175) (width 1) (layer "B.Cu") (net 7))
 (segment (start 58.98 59.8175) (end 54.8625 55.7) (width 1) (layer "B.Cu") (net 7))
 (segment (start 54.8625 55.7) (end 54.8625 51.94) (width 1) (layer "B.Cu") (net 7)))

